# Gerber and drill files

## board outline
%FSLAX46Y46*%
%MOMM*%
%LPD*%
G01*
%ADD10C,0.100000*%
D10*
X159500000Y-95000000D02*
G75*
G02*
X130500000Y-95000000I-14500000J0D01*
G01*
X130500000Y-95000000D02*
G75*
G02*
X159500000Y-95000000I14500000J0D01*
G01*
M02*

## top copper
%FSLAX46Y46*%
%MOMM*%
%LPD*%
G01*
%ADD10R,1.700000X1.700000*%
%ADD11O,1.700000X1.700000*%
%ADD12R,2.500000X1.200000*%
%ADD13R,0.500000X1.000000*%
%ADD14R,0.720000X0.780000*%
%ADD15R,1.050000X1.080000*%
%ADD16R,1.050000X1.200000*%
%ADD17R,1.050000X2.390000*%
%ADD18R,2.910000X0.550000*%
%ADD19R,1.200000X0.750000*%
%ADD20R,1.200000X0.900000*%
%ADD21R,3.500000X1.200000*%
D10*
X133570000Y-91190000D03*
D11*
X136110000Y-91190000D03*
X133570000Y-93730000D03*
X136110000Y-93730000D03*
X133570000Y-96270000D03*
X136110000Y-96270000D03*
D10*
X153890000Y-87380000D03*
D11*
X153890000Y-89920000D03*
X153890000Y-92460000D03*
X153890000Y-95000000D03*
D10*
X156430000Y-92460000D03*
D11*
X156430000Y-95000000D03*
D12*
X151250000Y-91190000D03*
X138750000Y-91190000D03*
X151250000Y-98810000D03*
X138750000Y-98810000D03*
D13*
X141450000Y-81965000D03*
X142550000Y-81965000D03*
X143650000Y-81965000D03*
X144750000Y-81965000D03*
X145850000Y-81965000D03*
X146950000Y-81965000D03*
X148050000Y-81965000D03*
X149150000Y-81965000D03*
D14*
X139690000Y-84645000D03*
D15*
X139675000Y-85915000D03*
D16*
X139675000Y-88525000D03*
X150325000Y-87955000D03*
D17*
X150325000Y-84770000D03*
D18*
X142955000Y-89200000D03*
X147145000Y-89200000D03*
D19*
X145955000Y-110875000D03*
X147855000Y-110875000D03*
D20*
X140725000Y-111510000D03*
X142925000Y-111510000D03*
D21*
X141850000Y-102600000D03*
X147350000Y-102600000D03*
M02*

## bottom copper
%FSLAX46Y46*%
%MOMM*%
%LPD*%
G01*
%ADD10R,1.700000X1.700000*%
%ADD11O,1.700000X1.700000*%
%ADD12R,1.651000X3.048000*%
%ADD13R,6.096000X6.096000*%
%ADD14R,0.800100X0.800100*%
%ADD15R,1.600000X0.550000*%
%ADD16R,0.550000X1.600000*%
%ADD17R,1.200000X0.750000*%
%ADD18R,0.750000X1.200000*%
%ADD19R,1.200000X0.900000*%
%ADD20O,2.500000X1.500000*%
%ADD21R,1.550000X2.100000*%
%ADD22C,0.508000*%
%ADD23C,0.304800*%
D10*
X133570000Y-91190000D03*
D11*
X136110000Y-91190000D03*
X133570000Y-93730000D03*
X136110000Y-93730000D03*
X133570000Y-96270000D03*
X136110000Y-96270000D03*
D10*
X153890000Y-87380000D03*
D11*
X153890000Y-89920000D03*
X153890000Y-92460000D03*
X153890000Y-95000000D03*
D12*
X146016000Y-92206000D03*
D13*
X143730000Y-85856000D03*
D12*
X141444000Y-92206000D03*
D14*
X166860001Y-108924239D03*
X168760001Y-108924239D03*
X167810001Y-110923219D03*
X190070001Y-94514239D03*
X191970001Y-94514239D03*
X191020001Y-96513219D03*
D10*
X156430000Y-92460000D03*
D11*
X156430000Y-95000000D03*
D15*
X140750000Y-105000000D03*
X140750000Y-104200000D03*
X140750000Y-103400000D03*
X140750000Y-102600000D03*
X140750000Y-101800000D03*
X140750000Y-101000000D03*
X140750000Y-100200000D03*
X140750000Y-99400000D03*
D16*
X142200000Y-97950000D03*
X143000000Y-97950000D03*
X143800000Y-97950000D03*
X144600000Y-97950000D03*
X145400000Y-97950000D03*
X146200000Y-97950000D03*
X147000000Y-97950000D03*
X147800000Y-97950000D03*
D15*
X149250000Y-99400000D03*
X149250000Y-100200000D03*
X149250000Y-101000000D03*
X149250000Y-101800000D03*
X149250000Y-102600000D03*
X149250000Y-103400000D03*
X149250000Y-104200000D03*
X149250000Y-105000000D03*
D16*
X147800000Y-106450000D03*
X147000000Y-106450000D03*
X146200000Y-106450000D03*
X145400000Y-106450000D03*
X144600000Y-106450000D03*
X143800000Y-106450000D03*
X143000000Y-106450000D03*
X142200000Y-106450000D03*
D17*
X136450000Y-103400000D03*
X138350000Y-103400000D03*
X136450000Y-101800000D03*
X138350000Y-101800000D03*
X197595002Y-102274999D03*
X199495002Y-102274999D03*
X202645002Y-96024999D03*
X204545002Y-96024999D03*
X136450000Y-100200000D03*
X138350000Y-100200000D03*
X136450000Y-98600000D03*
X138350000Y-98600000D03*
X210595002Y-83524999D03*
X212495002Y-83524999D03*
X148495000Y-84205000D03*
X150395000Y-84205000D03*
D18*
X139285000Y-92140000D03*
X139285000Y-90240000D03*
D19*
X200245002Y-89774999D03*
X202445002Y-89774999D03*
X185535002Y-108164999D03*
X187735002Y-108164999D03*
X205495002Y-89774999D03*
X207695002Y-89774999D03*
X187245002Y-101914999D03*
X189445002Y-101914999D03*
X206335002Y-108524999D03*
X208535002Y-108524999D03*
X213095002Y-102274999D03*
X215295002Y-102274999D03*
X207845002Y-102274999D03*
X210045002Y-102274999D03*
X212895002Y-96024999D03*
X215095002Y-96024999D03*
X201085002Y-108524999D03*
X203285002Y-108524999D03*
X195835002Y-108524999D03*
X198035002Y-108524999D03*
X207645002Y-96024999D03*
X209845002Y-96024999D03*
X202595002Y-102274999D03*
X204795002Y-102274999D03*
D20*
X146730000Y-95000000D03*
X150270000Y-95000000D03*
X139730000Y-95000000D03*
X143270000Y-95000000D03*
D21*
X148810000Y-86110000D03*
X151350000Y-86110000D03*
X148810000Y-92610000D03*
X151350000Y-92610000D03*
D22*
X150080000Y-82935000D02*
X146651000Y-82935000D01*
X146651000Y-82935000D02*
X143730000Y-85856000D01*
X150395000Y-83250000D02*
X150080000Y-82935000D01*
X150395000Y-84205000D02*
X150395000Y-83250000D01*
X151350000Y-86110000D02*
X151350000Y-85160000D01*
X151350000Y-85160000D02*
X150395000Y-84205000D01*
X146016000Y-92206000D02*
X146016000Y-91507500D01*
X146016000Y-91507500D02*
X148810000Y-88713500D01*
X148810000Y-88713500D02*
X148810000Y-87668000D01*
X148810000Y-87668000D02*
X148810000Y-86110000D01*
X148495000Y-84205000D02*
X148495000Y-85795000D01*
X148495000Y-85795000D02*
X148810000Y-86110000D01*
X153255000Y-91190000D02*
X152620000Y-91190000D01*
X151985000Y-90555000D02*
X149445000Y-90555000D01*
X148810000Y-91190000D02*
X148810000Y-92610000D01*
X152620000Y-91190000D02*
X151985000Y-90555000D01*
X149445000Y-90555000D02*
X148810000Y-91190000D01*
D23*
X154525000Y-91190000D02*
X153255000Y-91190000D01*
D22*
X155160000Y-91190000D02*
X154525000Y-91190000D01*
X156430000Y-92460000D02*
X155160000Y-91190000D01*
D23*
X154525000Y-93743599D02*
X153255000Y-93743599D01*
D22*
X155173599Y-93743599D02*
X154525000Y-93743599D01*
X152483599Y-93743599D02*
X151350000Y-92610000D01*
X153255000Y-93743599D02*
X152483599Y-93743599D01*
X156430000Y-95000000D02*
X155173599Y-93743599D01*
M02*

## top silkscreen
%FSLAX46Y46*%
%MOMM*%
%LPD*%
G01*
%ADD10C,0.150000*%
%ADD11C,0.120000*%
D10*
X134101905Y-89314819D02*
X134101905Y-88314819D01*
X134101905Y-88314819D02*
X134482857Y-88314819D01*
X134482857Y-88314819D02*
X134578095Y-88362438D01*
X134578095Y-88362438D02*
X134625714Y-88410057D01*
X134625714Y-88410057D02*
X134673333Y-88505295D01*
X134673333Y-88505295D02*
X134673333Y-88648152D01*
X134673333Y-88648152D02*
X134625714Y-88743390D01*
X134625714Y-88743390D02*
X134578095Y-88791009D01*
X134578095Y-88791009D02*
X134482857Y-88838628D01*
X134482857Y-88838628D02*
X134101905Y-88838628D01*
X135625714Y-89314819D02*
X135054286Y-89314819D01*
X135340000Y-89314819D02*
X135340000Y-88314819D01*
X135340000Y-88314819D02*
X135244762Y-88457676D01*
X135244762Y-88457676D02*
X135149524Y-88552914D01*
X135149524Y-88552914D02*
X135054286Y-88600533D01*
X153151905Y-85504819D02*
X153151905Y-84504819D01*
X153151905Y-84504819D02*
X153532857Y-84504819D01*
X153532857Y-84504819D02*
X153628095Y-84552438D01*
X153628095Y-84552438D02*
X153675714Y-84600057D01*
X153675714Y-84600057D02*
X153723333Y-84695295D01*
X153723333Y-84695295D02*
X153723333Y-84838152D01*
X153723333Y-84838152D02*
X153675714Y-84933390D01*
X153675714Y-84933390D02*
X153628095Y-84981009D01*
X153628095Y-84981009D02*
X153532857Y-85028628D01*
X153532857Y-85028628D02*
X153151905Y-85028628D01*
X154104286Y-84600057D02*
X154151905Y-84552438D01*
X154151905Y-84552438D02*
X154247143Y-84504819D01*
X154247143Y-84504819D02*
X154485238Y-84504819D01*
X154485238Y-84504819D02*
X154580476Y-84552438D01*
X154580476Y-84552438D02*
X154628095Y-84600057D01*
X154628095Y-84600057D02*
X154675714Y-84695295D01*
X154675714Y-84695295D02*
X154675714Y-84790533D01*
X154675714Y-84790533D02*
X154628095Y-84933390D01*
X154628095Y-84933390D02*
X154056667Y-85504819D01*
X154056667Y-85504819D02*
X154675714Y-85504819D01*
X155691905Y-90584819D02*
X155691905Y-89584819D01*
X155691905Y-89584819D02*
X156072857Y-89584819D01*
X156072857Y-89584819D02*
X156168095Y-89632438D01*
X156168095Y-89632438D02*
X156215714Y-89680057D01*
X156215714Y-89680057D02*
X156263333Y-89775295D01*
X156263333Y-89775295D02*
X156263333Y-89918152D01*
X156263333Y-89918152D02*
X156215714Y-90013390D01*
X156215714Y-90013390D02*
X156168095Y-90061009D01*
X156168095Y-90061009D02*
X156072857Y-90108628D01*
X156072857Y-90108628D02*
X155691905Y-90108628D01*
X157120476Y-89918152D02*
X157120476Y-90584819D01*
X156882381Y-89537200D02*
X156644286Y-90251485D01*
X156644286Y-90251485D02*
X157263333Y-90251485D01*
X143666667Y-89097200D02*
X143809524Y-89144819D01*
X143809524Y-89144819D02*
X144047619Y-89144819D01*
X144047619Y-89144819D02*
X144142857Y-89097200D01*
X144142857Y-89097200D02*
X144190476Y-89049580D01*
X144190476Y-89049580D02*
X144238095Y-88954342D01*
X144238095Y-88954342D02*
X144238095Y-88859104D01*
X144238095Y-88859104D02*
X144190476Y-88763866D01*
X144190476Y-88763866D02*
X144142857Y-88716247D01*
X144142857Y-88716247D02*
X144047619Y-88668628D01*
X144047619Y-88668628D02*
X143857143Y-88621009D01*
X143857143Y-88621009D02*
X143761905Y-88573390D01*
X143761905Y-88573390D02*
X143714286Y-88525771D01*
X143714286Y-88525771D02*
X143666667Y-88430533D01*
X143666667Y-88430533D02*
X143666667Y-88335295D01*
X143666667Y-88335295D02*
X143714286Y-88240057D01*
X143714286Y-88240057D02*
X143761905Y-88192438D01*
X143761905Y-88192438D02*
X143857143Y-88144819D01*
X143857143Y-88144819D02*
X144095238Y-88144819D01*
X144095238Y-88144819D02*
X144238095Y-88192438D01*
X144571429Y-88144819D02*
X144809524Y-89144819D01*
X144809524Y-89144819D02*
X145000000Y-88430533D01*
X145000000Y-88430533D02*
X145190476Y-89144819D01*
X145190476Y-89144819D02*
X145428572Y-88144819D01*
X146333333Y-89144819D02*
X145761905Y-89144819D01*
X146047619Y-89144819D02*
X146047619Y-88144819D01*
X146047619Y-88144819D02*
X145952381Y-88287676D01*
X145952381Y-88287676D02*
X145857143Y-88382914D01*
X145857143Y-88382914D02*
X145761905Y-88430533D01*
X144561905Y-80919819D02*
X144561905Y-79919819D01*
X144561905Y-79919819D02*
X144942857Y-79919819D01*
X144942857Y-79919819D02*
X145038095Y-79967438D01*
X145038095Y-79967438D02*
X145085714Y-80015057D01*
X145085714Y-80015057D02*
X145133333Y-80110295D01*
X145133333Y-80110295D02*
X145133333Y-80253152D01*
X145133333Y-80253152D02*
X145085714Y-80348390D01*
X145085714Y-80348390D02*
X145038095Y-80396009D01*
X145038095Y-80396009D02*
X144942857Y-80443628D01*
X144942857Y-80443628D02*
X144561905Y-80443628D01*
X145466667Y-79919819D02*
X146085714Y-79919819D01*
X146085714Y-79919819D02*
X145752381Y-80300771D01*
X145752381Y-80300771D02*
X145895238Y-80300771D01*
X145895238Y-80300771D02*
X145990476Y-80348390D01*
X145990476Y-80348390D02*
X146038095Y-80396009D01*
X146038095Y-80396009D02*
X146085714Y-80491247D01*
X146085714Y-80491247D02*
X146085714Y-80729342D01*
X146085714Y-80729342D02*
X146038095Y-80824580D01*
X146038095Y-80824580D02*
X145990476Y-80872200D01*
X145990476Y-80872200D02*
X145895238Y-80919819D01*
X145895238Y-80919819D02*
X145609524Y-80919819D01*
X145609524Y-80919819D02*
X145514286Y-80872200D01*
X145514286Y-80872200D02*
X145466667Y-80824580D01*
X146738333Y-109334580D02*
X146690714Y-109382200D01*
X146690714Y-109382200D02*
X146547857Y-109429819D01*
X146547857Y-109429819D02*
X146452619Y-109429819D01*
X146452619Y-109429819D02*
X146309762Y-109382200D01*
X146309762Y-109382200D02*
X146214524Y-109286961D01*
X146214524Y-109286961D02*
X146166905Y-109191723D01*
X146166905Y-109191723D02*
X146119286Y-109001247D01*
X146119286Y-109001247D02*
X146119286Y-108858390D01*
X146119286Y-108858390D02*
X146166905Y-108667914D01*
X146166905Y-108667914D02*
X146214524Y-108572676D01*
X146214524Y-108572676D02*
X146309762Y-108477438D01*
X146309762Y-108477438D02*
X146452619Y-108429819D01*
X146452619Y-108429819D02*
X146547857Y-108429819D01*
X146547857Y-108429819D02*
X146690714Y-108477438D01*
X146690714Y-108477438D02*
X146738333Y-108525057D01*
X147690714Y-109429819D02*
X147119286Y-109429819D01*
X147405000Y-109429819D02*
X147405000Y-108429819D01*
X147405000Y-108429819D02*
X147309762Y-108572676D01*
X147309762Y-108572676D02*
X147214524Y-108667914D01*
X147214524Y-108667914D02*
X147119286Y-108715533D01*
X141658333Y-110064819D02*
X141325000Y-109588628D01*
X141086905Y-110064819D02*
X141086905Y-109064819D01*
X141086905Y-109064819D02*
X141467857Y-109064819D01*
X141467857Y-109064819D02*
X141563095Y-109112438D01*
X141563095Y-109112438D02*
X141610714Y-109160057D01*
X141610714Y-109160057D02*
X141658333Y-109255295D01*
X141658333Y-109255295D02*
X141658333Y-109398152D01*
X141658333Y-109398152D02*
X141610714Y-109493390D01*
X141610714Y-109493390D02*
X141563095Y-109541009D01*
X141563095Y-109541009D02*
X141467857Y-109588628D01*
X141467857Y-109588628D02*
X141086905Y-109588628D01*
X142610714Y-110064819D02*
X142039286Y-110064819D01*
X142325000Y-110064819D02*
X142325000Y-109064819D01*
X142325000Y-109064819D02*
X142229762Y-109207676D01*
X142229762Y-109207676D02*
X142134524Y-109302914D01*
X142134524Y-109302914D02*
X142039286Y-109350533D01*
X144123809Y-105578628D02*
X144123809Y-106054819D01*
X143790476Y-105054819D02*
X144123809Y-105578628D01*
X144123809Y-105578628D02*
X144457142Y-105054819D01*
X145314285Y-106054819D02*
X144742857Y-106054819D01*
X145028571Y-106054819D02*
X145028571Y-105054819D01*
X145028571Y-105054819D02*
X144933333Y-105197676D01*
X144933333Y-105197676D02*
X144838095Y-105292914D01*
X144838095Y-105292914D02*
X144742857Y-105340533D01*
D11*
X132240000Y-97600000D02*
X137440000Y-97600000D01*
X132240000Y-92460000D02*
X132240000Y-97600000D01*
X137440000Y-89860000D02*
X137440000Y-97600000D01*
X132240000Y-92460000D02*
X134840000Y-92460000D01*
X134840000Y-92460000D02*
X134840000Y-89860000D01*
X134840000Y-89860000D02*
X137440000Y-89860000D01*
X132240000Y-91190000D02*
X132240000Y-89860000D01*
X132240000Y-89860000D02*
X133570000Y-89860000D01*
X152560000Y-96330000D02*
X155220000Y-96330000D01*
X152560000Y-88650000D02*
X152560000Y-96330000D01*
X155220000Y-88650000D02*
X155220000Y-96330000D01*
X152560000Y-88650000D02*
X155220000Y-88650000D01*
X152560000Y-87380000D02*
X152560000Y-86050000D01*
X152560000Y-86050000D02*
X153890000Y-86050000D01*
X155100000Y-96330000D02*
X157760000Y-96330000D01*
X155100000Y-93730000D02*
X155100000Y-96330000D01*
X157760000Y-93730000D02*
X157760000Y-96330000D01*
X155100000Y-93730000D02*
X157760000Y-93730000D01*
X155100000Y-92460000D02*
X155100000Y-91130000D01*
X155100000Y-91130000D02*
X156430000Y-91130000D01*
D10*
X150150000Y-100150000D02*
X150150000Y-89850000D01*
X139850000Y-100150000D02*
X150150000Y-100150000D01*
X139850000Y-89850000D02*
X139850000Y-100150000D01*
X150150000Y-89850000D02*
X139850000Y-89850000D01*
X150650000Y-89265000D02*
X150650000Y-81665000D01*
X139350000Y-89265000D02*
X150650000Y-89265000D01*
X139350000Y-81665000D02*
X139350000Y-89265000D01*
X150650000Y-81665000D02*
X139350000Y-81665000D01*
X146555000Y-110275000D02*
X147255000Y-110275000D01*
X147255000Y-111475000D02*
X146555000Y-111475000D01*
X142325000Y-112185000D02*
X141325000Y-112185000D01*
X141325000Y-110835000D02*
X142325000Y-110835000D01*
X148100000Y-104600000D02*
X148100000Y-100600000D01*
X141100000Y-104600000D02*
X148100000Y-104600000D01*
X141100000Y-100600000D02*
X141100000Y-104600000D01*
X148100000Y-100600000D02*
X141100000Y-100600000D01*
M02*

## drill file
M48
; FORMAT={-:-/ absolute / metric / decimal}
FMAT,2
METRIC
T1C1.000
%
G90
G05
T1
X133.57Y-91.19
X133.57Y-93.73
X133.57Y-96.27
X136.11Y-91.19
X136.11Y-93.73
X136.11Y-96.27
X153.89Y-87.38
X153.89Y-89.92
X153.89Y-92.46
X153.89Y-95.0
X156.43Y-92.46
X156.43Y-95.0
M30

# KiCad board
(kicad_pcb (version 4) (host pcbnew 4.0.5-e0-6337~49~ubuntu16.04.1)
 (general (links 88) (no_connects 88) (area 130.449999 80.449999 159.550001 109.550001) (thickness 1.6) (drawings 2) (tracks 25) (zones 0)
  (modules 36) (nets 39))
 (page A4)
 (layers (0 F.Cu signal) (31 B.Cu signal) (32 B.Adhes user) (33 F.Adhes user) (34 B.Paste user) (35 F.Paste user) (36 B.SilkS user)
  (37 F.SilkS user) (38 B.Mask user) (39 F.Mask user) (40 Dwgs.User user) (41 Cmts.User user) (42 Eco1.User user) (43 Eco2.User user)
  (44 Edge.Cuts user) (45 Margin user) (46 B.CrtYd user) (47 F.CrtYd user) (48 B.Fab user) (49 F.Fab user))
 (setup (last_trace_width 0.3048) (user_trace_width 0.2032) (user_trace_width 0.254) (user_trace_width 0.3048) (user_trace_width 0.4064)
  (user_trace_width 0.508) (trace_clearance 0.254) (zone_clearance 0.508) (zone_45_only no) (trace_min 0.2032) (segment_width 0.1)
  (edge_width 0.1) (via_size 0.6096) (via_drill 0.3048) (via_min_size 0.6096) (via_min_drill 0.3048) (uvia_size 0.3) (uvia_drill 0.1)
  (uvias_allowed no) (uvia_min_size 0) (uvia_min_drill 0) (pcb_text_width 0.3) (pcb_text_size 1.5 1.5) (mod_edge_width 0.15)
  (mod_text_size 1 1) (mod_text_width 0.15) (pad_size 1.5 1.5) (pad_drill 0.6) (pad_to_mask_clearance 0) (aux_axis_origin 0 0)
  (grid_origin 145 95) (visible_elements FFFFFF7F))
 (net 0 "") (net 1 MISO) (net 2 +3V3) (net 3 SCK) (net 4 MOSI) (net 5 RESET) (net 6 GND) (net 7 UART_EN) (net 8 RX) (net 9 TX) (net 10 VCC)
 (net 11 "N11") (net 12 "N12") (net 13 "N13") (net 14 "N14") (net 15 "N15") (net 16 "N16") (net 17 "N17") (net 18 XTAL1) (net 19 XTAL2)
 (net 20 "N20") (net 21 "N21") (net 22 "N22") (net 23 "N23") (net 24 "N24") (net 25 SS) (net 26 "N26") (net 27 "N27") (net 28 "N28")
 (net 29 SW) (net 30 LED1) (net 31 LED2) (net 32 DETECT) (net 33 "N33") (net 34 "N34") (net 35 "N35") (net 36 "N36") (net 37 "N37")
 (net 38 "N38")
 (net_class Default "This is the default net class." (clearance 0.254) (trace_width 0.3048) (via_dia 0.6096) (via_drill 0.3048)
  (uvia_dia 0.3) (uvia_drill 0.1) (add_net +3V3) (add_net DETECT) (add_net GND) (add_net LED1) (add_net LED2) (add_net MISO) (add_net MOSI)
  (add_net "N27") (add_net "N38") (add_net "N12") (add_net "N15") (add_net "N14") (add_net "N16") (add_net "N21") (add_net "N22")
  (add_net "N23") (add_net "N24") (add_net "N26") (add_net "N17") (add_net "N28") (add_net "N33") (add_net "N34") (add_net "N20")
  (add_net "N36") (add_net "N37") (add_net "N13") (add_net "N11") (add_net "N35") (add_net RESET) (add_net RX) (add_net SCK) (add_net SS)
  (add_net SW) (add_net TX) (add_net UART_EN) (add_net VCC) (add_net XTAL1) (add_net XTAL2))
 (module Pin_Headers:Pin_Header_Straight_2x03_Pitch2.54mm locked (layer F.Cu) (at 133.57 91.19)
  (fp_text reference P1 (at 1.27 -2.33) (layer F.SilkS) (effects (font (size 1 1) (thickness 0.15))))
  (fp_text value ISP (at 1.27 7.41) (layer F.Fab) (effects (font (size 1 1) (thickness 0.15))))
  (fp_line (start -1.33 6.41) (end 3.87 6.41) (layer F.SilkS) (width 0.12))
  (fp_line (start -1.33 1.27) (end -1.33 6.41) (layer F.SilkS) (width 0.12))
  (fp_line (start 3.87 -1.33) (end 3.87 6.41) (layer F.SilkS) (width 0.12))
  (fp_line (start -1.33 1.27) (end 1.27 1.27) (layer F.SilkS) (width 0.12))
  (fp_line (start 1.27 1.27) (end 1.27 -1.33) (layer F.SilkS) (width 0.12))
  (fp_line (start 1.27 -1.33) (end 3.87 -1.33) (layer F.SilkS) (width 0.12))
  (fp_line (start -1.33 0) (end -1.33 -1.33) (layer F.SilkS) (width 0.12))
  (fp_line (start -1.33 -1.33) (end 0 -1.33) (layer F.SilkS) (width 0.12))
  (pad 1 thru_hole rect (at 0 0) (size 1.7 1.7) (drill 1) (layers *.Cu *.Mask) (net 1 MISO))
  (pad 2 thru_hole oval (at 2.54 0) (size 1.7 1.7) (drill 1) (layers *.Cu *.Mask) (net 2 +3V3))
  (pad 3 thru_hole oval (at 0 2.54) (size 1.7 1.7) (drill 1) (layers *.Cu *.Mask) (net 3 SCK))
  (pad 4 thru_hole oval (at 2.54 2.54) (size 1.7 1.7) (drill 1) (layers *.Cu *.Mask) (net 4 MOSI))
  (pad 5 thru_hole oval (at 0 5.08) (size 1.7 1.7) (drill 1) (layers *.Cu *.Mask) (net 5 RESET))
  (pad 6 thru_hole oval (at 2.54 5.08) (size 1.7 1.7) (drill 1) (layers *.Cu *.Mask) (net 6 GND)))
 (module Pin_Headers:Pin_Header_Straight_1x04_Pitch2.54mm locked (layer F.Cu) (at 153.89 87.38)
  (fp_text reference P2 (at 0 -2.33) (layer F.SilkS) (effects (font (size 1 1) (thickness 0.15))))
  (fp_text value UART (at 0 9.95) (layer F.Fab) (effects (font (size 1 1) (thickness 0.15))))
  (fp_line (start -1.33 8.95) (end 1.33 8.95) (layer F.SilkS) (width 0.12))
  (fp_line (start -1.33 1.27) (end -1.33 8.95) (layer F.SilkS) (width 0.12))
  (fp_line (start 1.33 1.27) (end 1.33 8.95) (layer F.SilkS) (width 0.12))
  (fp_line (start -1.33 1.27) (end 1.33 1.27) (layer F.SilkS) (width 0.12))
  (fp_line (start -1.33 0) (end -1.33 -1.33) (layer F.SilkS) (width 0.12))
  (fp_line (start -1.33 -1.33) (end 0 -1.33) (layer F.SilkS) (width 0.12))
  (pad 1 thru_hole rect (at 0 0) (size 1.7 1.7) (drill 1) (layers *.Cu *.Mask) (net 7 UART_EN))
  (pad 2 thru_hole oval (at 0 2.54) (size 1.7 1.7) (drill 1) (layers *.Cu *.Mask) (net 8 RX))
  (pad 3 thru_hole oval (at 0 5.08) (size 1.7 1.7) (drill 1) (layers *.Cu *.Mask) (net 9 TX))
  (pad 4 thru_hole oval (at 0 7.62) (size 1.7 1.7) (drill 1) (layers *.Cu *.Mask) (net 6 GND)))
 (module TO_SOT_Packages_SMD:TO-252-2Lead (layer B.Cu) (at 143.73 92.206 180)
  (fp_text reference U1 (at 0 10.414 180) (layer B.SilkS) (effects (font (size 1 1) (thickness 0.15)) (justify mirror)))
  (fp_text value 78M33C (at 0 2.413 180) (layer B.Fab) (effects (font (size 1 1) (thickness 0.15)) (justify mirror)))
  (pad 1 smd rect (at -2.286 0 180) (size 1.651 3.048) (layers B.Cu B.Paste B.Mask) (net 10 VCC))
  (pad 2 smd rect (at 0 6.35 180) (size 6.096 6.096) (layers B.Cu B.Paste B.Mask) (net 6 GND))
  (pad 3 smd rect (at 2.286 0 180) (size 1.651 3.048) (layers B.Cu B.Paste B.Mask) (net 2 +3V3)))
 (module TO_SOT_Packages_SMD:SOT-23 (layer B.Cu) (at 167.810001 109.924999)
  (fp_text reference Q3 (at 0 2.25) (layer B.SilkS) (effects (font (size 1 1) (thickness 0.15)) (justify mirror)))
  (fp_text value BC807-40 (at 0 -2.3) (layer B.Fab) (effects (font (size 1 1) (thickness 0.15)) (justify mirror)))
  (pad 1 smd rect (at -0.95 -1.00076) (size 0.8001 0.8001) (layers B.Cu B.Paste B.Mask) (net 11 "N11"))
  (pad 2 smd rect (at 0.95 -1.00076) (size 0.8001 0.8001) (layers B.Cu B.Paste B.Mask) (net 2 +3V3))
  (pad 3 smd rect (at 0 0.99822) (size 0.8001 0.8001) (layers B.Cu B.Paste B.Mask) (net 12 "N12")))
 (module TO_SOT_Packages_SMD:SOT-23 (layer B.Cu) (at 191.020001 95.514999)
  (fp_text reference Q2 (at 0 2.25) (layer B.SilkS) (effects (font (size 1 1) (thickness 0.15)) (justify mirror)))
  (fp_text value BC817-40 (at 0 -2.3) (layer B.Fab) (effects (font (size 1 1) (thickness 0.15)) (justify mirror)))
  (pad 1 smd rect (at -0.95 -1.00076) (size 0.8001 0.8001) (layers B.Cu B.Paste B.Mask) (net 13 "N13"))
  (pad 2 smd rect (at 0.95 -1.00076) (size 0.8001 0.8001) (layers B.Cu B.Paste B.Mask) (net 6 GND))
  (pad 3 smd rect (at 0 0.99822) (size 0.8001 0.8001) (layers B.Cu B.Paste B.Mask) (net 8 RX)))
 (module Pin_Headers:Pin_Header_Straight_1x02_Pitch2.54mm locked (layer F.Cu) (at 156.43 92.46)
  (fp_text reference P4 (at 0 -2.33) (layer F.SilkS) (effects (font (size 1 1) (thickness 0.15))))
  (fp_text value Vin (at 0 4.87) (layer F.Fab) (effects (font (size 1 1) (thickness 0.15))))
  (fp_line (start -1.33 3.87) (end 1.33 3.87) (layer F.SilkS) (width 0.12))
  (fp_line (start -1.33 1.27) (end -1.33 3.87) (layer F.SilkS) (width 0.12))
  (fp_line (start 1.33 1.27) (end 1.33 3.87) (layer F.SilkS) (width 0.12))
  (fp_line (start -1.33 1.27) (end 1.33 1.27) (layer F.SilkS) (width 0.12))
  (fp_line (start -1.33 0) (end -1.33 -1.33) (layer F.SilkS) (width 0.12))
  (fp_line (start -1.33 -1.33) (end 0 -1.33) (layer F.SilkS) (width 0.12))
  (pad 1 thru_hole rect (at 0 0) (size 1.7 1.7) (drill 1) (layers *.Cu *.Mask) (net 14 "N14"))
  (pad 2 thru_hole oval (at 0 2.54) (size 1.7 1.7) (drill 1) (layers *.Cu *.Mask) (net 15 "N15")))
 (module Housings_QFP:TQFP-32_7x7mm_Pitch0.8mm (layer B.Cu) (at 145 102.2)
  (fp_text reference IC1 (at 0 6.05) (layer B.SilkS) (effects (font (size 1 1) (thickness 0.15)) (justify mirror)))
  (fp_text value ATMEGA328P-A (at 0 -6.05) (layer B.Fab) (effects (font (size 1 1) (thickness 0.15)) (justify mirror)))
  (pad 1 smd rect (at -4.25 2.8) (size 1.6 0.55) (layers B.Cu B.Paste B.Mask) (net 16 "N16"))
  (pad 2 smd rect (at -4.25 2) (size 1.6 0.55) (layers B.Cu B.Paste B.Mask) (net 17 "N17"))
  (pad 3 smd rect (at -4.25 1.2) (size 1.6 0.55) (layers B.Cu B.Paste B.Mask) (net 6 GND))
  (pad 4 smd rect (at -4.25 0.4) (size 1.6 0.55) (layers B.Cu B.Paste B.Mask) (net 2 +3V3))
  (pad 5 smd rect (at -4.25 -0.4) (size 1.6 0.55) (layers B.Cu B.Paste B.Mask) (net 6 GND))
  (pad 6 smd rect (at -4.25 -1.2) (size 1.6 0.55) (layers B.Cu B.Paste B.Mask) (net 2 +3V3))
  (pad 7 smd rect (at -4.25 -2) (size 1.6 0.55) (layers B.Cu B.Paste B.Mask) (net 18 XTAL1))
  (pad 8 smd rect (at -4.25 -2.8) (size 1.6 0.55) (layers B.Cu B.Paste B.Mask) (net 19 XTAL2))
  (pad 9 smd rect (at -2.8 -4.25 270) (size 1.6 0.55) (layers B.Cu B.Paste B.Mask) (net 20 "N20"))
  (pad 10 smd rect (at -2 -4.25 270) (size 1.6 0.55) (layers B.Cu B.Paste B.Mask) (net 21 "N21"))
  (pad 11 smd rect (at -1.2 -4.25 270) (size 1.6 0.55) (layers B.Cu B.Paste B.Mask) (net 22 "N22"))
  (pad 12 smd rect (at -0.4 -4.25 270) (size 1.6 0.55) (layers B.Cu B.Paste B.Mask) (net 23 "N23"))
  (pad 13 smd rect (at 0.4 -4.25 270) (size 1.6 0.55) (layers B.Cu B.Paste B.Mask) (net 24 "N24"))
  (pad 14 smd rect (at 1.2 -4.25 270) (size 1.6 0.55) (layers B.Cu B.Paste B.Mask) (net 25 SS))
  (pad 15 smd rect (at 2 -4.25 270) (size 1.6 0.55) (layers B.Cu B.Paste B.Mask) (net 4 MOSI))
  (pad 16 smd rect (at 2.8 -4.25 270) (size 1.6 0.55) (layers B.Cu B.Paste B.Mask) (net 1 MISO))
  (pad 17 smd rect (at 4.25 -2.8) (size 1.6 0.55) (layers B.Cu B.Paste B.Mask) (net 3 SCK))
  (pad 18 smd rect (at 4.25 -2) (size 1.6 0.55) (layers B.Cu B.Paste B.Mask) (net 2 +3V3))
  (pad 19 smd rect (at 4.25 -1.2) (size 1.6 0.55) (layers B.Cu B.Paste B.Mask) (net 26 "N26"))
  (pad 20 smd rect (at 4.25 -0.4) (size 1.6 0.55) (layers B.Cu B.Paste B.Mask) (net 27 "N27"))
  (pad 21 smd rect (at 4.25 0.4) (size 1.6 0.55) (layers B.Cu B.Paste B.Mask) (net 6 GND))
  (pad 22 smd rect (at 4.25 1.2) (size 1.6 0.55) (layers B.Cu B.Paste B.Mask) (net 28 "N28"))
  (pad 23 smd rect (at 4.25 2) (size 1.6 0.55) (layers B.Cu B.Paste B.Mask) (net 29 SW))
  (pad 24 smd rect (at 4.25 2.8) (size 1.6 0.55) (layers B.Cu B.Paste B.Mask) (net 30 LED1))
  (pad 25 smd rect (at 2.8 4.25 270) (size 1.6 0.55) (layers B.Cu B.Paste B.Mask) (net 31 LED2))
  (pad 26 smd rect (at 2 4.25 270) (size 1.6 0.55) (layers B.Cu B.Paste B.Mask) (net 7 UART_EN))
  (pad 27 smd rect (at 1.2 4.25 270) (size 1.6 0.55) (layers B.Cu B.Paste B.Mask) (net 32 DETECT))
  (pad 28 smd rect (at 0.4 4.25 270) (size 1.6 0.55) (layers B.Cu B.Paste B.Mask) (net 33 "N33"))
  (pad 29 smd rect (at -0.4 4.25 270) (size 1.6 0.55) (layers B.Cu B.Paste B.Mask) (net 5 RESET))
  (pad 30 smd rect (at -1.2 4.25 270) (size 1.6 0.55) (layers B.Cu B.Paste B.Mask) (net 8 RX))
  (pad 31 smd rect (at -2 4.25 270) (size 1.6 0.55) (layers B.Cu B.Paste B.Mask) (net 9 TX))
  (pad 32 smd rect (at -2.8 4.25 270) (size 1.6 0.55) (layers B.Cu B.Paste B.Mask) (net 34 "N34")))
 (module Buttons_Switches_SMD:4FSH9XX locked (layer F.Cu) (at 145 95)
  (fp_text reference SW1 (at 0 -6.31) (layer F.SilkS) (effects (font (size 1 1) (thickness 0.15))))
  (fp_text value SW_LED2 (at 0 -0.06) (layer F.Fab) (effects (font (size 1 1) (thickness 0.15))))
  (fp_line (start 5.15 5.15) (end 5.15 -5.15) (layer F.SilkS) (width 0.15))
  (fp_line (start -5.15 5.15) (end 5.15 5.15) (layer F.SilkS) (width 0.15))
  (fp_line (start -5.15 -5.15) (end -5.15 5.15) (layer F.SilkS) (width 0.15))
  (fp_line (start 5.15 -5.15) (end -5.15 -5.15) (layer F.SilkS) (width 0.15))
  (pad 1 smd rect (at 6.25 -3.81) (size 2.5 1.2) (layers F.Cu F.Paste F.Mask) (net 29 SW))
  (pad 2 smd rect (at -6.25 -3.81) (size 2.5 1.2) (layers F.Cu F.Paste F.Mask) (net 31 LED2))
  (pad 3 smd rect (at 6.25 3.81) (size 2.5 1.2) (layers F.Cu F.Paste F.Mask) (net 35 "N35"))
  (pad 4 smd rect (at -6.25 3.81) (size 2.5 1.2) (layers F.Cu F.Paste F.Mask) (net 6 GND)))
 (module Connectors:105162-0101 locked (layer F.Cu) (at 145 81.665 180)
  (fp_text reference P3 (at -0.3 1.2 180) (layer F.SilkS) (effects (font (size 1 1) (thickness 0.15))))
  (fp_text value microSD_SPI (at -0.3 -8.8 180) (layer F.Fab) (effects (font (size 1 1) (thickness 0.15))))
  (fp_line (start -5.65 -7.6) (end -5.65 0) (layer F.SilkS) (width 0.15))
  (fp_line (start 5.65 -7.6) (end -5.65 -7.6) (layer F.SilkS) (width 0.15))
  (fp_line (start 5.65 0) (end 5.65 -7.6) (layer F.SilkS) (width 0.15))
  (fp_line (start -5.65 0) (end 5.65 0) (layer F.SilkS) (width 0.15))
  (pad 1 smd rect (at 3.55 -0.3 180) (size 0.5 1) (layers F.Cu F.Paste F.Mask) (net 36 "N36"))
  (pad 2 smd rect (at 2.45 -0.3 180) (size 0.5 1) (layers F.Cu F.Paste F.Mask) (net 25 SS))
  (pad 3 smd rect (at 1.35 -0.3 180) (size 0.5 1) (layers F.Cu F.Paste F.Mask) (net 4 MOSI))
  (pad 4 smd rect (at 0.25 -0.3 180) (size 0.5 1) (layers F.Cu F.Paste F.Mask) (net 2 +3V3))
  (pad 5 smd rect (at -0.85 -0.3 180) (size 0.5 1) (layers F.Cu F.Paste F.Mask) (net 3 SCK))
  (pad 6 smd rect (at -1.95 -0.3 180) (size 0.5 1) (layers F.Cu F.Paste F.Mask) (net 6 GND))
  (pad 7 smd rect (at -3.05 -0.3 180) (size 0.5 1) (layers F.Cu F.Paste F.Mask) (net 1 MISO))
  (pad 8 smd rect (at -4.15 -0.3 180) (size 0.5 1) (layers F.Cu F.Paste F.Mask) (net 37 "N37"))
  (pad 9 smd rect (at 5.31 -2.98 180) (size 0.72 0.78) (layers F.Cu F.Paste F.Mask) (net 32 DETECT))
  (pad G1 smd rect (at 5.325 -4.25 180) (size 1.05 1.08) (layers F.Cu F.Paste F.Mask) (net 6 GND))
  (pad G2 smd rect (at 5.325 -6.86 180) (size 1.05 1.2) (layers F.Cu F.Paste F.Mask) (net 6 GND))
  (pad G3 smd rect (at -5.325 -6.29 180) (size 1.05 1.2) (layers F.Cu F.Paste F.Mask) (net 6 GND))
  (pad G4 smd rect (at -5.325 -3.105 180) (size 1.05 2.39) (layers F.Cu F.Paste F.Mask) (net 6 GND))
  (pad "" smd rect (at 2.045 -7.535 180) (size 2.91 0.55) (layers F.Cu F.Paste F.Mask))
  (pad "" smd rect (at -2.145 -7.535 180) (size 2.91 0.55) (layers F.Cu F.Paste F.Mask)))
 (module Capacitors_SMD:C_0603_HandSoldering (layer F.Cu) (at 146.905 110.875)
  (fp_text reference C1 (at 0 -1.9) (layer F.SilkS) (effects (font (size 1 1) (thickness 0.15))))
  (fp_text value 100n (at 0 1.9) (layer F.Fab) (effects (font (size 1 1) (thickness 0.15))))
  (fp_line (start -0.35 -0.6) (end 0.35 -0.6) (layer F.SilkS) (width 0.15))
  (fp_line (start 0.35 0.6) (end -0.35 0.6) (layer F.SilkS) (width 0.15))
  (pad 1 smd rect (at -0.95 0) (size 1.2 0.75) (layers F.Cu F.Paste F.Mask) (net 5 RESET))
  (pad 2 smd rect (at 0.95 0) (size 1.2 0.75) (layers F.Cu F.Paste F.Mask) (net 6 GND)))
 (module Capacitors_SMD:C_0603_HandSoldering (layer B.Cu) (at 137.4 103.4)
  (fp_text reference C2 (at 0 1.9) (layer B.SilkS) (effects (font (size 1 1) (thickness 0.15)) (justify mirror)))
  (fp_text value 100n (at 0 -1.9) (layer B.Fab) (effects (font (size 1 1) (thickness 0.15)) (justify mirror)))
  (pad 1 smd rect (at -0.95 0) (size 1.2 0.75) (layers B.Cu B.Paste B.Mask) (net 2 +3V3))
  (pad 2 smd rect (at 0.95 0) (size 1.2 0.75) (layers B.Cu B.Paste B.Mask) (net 6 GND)))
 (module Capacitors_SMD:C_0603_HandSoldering (layer B.Cu) (at 137.4 101.8)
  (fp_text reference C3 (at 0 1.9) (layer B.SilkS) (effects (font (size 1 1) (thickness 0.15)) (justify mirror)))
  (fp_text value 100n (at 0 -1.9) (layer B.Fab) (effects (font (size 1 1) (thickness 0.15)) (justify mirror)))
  (pad 1 smd rect (at -0.95 0) (size 1.2 0.75) (layers B.Cu B.Paste B.Mask) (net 2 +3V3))
  (pad 2 smd rect (at 0.95 0) (size 1.2 0.75) (layers B.Cu B.Paste B.Mask) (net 6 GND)))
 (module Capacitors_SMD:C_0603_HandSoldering (layer B.Cu) (at 198.545002 102.274999)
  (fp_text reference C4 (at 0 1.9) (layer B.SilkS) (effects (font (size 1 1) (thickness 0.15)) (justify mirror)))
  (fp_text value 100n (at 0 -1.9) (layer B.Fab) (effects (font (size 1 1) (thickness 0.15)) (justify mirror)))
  (pad 1 smd rect (at -0.95 0) (size 1.2 0.75) (layers B.Cu B.Paste B.Mask) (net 2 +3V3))
  (pad 2 smd rect (at 0.95 0) (size 1.2 0.75) (layers B.Cu B.Paste B.Mask) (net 6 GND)))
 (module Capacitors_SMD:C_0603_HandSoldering (layer B.Cu) (at 203.595002 96.024999)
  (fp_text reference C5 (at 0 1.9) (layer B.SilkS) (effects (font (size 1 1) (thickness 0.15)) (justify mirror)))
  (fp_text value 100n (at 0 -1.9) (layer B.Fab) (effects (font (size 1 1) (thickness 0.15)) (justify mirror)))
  (pad 1 smd rect (at -0.95 0) (size 1.2 0.75) (layers B.Cu B.Paste B.Mask) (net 27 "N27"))
  (pad 2 smd rect (at 0.95 0) (size 1.2 0.75) (layers B.Cu B.Paste B.Mask) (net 6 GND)))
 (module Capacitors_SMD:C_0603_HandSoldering (layer B.Cu) (at 137.4 100.2)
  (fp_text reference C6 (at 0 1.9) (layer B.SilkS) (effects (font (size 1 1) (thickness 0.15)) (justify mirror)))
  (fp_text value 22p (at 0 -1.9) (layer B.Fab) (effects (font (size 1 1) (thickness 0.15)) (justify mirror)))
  (pad 1 smd rect (at -0.95 0) (size 1.2 0.75) (layers B.Cu B.Paste B.Mask) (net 6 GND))
  (pad 2 smd rect (at 0.95 0) (size 1.2 0.75) (layers B.Cu B.Paste B.Mask) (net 18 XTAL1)))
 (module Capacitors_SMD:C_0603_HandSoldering (layer B.Cu) (at 137.4 98.6)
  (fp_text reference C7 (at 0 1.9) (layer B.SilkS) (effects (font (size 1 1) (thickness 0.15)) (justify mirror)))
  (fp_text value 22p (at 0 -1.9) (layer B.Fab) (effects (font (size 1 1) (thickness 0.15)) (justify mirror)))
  (pad 1 smd rect (at -0.95 0) (size 1.2 0.75) (layers B.Cu B.Paste B.Mask) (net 6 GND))
  (pad 2 smd rect (at 0.95 0) (size 1.2 0.75) (layers B.Cu B.Paste B.Mask) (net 19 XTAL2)))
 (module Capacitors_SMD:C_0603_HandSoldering (layer B.Cu) (at 211.545002 83.524999)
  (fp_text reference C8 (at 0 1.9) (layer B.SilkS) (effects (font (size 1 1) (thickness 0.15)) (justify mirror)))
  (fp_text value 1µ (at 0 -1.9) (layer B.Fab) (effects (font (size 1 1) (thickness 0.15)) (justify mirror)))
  (pad 1 smd rect (at -0.95 0) (size 1.2 0.75) (layers B.Cu B.Paste B.Mask) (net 2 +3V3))
  (pad 2 smd rect (at 0.95 0) (size 1.2 0.75) (layers B.Cu B.Paste B.Mask) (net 6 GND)))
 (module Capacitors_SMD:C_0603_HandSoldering (layer B.Cu) (at 149.445 84.205)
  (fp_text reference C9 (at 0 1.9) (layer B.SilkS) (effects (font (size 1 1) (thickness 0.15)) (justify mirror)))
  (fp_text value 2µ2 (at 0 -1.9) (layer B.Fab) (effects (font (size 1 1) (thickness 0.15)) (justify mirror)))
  (pad 1 smd rect (at -0.95 0) (size 1.2 0.75) (layers B.Cu B.Paste B.Mask) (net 10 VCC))
  (pad 2 smd rect (at 0.95 0) (size 1.2 0.75) (layers B.Cu B.Paste B.Mask) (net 6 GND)))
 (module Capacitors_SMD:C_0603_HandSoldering (layer B.Cu) (at 139.285 91.19 90)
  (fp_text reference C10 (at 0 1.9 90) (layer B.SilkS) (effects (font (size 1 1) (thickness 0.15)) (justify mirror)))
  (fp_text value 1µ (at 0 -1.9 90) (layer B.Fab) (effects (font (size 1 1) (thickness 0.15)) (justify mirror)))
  (pad 1 smd rect (at -0.95 0 90) (size 1.2 0.75) (layers B.Cu B.Paste B.Mask) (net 2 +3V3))
  (pad 2 smd rect (at 0.95 0 90) (size 1.2 0.75) (layers B.Cu B.Paste B.Mask) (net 6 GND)))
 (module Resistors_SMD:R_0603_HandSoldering (layer F.Cu) (at 141.825 111.51)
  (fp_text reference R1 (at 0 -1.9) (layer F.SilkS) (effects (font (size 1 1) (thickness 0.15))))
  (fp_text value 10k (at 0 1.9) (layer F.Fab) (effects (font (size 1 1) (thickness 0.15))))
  (fp_line (start 0.5 0.675) (end -0.5 0.675) (layer F.SilkS) (width 0.15))
  (fp_line (start -0.5 -0.675) (end 0.5 -0.675) (layer F.SilkS) (width 0.15))
  (pad 1 smd rect (at -1.1 0) (size 1.2 0.9) (layers F.Cu F.Paste F.Mask) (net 2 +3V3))
  (pad 2 smd rect (at 1.1 0) (size 1.2 0.9) (layers F.Cu F.Paste F.Mask) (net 5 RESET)))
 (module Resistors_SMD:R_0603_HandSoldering (layer B.Cu) (at 201.345002 89.774999)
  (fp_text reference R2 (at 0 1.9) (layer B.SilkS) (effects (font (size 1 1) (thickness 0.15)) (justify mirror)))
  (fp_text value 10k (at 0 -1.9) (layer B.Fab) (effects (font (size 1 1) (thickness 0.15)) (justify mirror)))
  (pad 1 smd rect (at -1.1 0) (size 1.2 0.9) (layers B.Cu B.Paste B.Mask) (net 2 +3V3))
  (pad 2 smd rect (at 1.1 0) (size 1.2 0.9) (layers B.Cu B.Paste B.Mask) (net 7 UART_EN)))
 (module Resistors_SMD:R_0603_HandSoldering (layer B.Cu) (at 186.635002 108.164999)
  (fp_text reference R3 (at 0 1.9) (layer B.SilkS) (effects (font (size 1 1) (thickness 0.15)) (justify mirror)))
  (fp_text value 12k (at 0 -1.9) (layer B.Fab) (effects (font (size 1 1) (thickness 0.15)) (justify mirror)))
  (pad 1 smd rect (at -1.1 0) (size 1.2 0.9) (layers B.Cu B.Paste B.Mask) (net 13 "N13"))
  (pad 2 smd rect (at 1.1 0) (size 1.2 0.9) (layers B.Cu B.Paste B.Mask) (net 6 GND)))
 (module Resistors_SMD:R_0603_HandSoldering (layer B.Cu) (at 206.595002 89.774999)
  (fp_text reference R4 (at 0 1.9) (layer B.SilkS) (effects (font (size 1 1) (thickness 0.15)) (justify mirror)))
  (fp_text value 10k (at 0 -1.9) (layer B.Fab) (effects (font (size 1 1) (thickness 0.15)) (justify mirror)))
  (pad 1 smd rect (at -1.1 0) (size 1.2 0.9) (layers B.Cu B.Paste B.Mask) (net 2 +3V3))
  (pad 2 smd rect (at 1.1 0) (size 1.2 0.9) (layers B.Cu B.Paste B.Mask) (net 1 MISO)))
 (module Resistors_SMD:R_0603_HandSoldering (layer B.Cu) (at 188.345002 101.914999)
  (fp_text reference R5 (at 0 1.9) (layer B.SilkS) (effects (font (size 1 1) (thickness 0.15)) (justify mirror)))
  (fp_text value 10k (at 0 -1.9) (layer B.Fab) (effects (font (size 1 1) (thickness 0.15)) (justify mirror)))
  (pad 1 smd rect (at -1.1 0) (size 1.2 0.9) (layers B.Cu B.Paste B.Mask) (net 2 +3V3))
  (pad 2 smd rect (at 1.1 0) (size 1.2 0.9) (layers B.Cu B.Paste B.Mask) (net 25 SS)))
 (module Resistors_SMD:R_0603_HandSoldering (layer B.Cu) (at 207.435002 108.524999)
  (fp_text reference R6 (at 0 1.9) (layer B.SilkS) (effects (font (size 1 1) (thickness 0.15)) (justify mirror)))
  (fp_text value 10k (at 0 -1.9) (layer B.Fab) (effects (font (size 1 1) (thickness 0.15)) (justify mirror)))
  (pad 1 smd rect (at -1.1 0) (size 1.2 0.9) (layers B.Cu B.Paste B.Mask) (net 2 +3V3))
  (pad 2 smd rect (at 1.1 0) (size 1.2 0.9) (layers B.Cu B.Paste B.Mask) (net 32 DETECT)))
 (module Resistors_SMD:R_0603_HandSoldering (layer B.Cu) (at 214.195002 102.274999)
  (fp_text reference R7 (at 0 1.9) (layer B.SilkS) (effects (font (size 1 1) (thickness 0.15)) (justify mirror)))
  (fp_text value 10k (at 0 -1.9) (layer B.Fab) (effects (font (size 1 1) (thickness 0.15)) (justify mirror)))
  (pad 1 smd rect (at -1.1 0) (size 1.2 0.9) (layers B.Cu B.Paste B.Mask) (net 2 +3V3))
  (pad 2 smd rect (at 1.1 0) (size 1.2 0.9) (layers B.Cu B.Paste B.Mask) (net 37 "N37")))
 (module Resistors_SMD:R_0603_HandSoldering (layer B.Cu) (at 208.945002 102.274999)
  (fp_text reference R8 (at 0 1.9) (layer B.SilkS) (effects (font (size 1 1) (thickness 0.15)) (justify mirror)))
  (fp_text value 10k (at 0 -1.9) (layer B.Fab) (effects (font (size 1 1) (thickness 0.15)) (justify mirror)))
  (pad 1 smd rect (at -1.1 0) (size 1.2 0.9) (layers B.Cu B.Paste B.Mask) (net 2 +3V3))
  (pad 2 smd rect (at 1.1 0) (size 1.2 0.9) (layers B.Cu B.Paste B.Mask) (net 36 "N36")))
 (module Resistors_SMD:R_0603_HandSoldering (layer B.Cu) (at 213.995002 96.024999)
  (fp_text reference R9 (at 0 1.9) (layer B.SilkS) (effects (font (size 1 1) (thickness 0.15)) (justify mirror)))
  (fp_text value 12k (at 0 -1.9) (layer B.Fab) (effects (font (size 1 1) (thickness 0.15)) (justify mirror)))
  (pad 1 smd rect (at -1.1 0) (size 1.2 0.9) (layers B.Cu B.Paste B.Mask) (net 2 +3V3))
  (pad 2 smd rect (at 1.1 0) (size 1.2 0.9) (layers B.Cu B.Paste B.Mask) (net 8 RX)))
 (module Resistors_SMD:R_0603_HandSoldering (layer B.Cu) (at 202.185002 108.524999)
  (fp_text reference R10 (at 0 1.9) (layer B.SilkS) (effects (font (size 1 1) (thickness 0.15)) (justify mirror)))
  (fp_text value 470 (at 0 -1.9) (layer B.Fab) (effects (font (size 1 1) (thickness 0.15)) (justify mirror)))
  (pad 1 smd rect (at -1.1 0) (size 1.2 0.9) (layers B.Cu B.Paste B.Mask) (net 30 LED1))
  (pad 2 smd rect (at 1.1 0) (size 1.2 0.9) (layers B.Cu B.Paste B.Mask) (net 35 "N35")))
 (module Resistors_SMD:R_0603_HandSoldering (layer B.Cu) (at 196.935002 108.524999)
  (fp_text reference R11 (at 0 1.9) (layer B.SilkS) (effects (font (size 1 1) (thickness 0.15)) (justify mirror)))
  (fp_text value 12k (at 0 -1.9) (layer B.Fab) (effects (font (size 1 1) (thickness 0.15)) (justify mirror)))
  (pad 1 smd rect (at -1.1 0) (size 1.2 0.9) (layers B.Cu B.Paste B.Mask) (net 11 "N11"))
  (pad 2 smd rect (at 1.1 0) (size 1.2 0.9) (layers B.Cu B.Paste B.Mask) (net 9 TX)))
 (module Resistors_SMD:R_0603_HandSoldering (layer B.Cu) (at 208.745002 96.024999)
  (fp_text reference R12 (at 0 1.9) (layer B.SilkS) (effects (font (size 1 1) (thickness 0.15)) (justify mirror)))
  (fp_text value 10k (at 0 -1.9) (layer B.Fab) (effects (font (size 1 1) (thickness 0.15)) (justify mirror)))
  (pad 1 smd rect (at -1.1 0) (size 1.2 0.9) (layers B.Cu B.Paste B.Mask) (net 2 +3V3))
  (pad 2 smd rect (at 1.1 0) (size 1.2 0.9) (layers B.Cu B.Paste B.Mask) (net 29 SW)))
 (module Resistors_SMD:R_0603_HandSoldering (layer B.Cu) (at 203.695002 102.274999)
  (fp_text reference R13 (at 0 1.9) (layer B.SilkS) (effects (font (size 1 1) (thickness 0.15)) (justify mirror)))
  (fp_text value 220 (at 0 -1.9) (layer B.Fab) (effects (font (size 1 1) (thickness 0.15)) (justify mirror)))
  (pad 1 smd rect (at -1.1 0) (size 1.2 0.9) (layers B.Cu B.Paste B.Mask) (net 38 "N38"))
  (pad 2 smd rect (at 1.1 0) (size 1.2 0.9) (layers B.Cu B.Paste B.Mask) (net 6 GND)))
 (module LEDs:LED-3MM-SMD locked (layer B.Cu) (at 148.5 95)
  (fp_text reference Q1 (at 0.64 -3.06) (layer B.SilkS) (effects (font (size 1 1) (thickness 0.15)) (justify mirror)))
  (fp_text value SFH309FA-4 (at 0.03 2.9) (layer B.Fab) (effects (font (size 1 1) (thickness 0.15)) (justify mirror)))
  (pad 1 smd oval (at -1.77 0 270) (size 1.5 2.5) (layers B.Cu B.Paste B.Mask) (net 2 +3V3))
  (pad 2 smd oval (at 1.77 0) (size 2.5 1.5) (layers B.Cu B.Paste B.Mask) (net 13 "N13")))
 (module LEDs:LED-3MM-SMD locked (layer B.Cu) (at 141.5 95)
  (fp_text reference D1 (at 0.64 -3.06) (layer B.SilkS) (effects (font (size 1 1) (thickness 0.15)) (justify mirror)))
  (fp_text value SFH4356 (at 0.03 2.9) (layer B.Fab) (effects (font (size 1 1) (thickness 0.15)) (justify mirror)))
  (pad 1 smd oval (at -1.77 0 270) (size 1.5 2.5) (layers B.Cu B.Paste B.Mask) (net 38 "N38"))
  (pad 2 smd oval (at 1.77 0) (size 2.5 1.5) (layers B.Cu B.Paste B.Mask) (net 12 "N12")))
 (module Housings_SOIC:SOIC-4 (layer B.Cu) (at 150.08 89.36)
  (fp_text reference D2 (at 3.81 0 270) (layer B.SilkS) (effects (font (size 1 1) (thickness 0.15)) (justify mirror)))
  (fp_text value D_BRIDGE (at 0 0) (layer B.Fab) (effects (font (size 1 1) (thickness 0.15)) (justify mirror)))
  (pad 1 smd rect (at -1.27 -3.25) (size 1.55 2.1) (layers B.Cu B.Paste B.Mask) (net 10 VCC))
  (pad 2 smd rect (at 1.27 -3.25) (size 1.55 2.1) (layers B.Cu B.Paste B.Mask) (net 6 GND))
  (pad 4 smd rect (at -1.27 3.25) (size 1.55 2.1) (layers B.Cu B.Paste B.Mask) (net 14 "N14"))
  (pad 3 smd rect (at 1.27 3.25) (size 1.55 2.1) (layers B.Cu B.Paste B.Mask) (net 15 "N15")))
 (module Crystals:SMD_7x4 (layer F.Cu) (at 144.6 102.6)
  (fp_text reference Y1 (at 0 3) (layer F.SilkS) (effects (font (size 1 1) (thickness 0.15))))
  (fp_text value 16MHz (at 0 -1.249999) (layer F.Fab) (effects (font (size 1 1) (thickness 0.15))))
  (fp_line (start 3.5 2) (end 3.5 -2) (layer F.SilkS) (width 0.15))
  (fp_line (start -3.5 2) (end 3.5 2) (layer F.SilkS) (width 0.15))
  (fp_line (start -3.5 -2) (end -3.5 2) (layer F.SilkS) (width 0.15))
  (fp_line (start 3.5 -2) (end -3.5 -2) (layer F.SilkS) (width 0.15))
  (pad 1 smd rect (at -2.75 0) (size 3.5 1.2) (layers F.Cu F.Paste F.Mask) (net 18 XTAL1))
  (pad 2 smd rect (at 2.75 0) (size 3.5 1.2) (layers F.Cu F.Paste F.Mask) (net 19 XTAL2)))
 (gr_circle (center 145 95) (end 159.5 95) (layer Edge.Cuts) (width 0.1))
 (segment (start 150.08 82.935) (end 146.651 82.935) (width 0.508) (layer B.Cu) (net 6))
 (segment (start 146.651 82.935) (end 143.73 85.856) (width 0.508) (layer B.Cu) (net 6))
 (segment (start 150.395 83.25) (end 150.08 82.935) (width 0.508) (layer B.Cu) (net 6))
 (segment (start 150.395 84.205) (end 150.395 83.25) (width 0.508) (layer B.Cu) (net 6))
 (segment (start 151.35 86.11) (end 151.35 85.16) (width 0.508) (layer B.Cu) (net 6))
 (segment (start 151.35 85.16) (end 150.395 84.205) (width 0.508) (layer B.Cu) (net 6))
 (segment (start 146.016 92.206) (end 146.016 91.5075) (width 0.508) (layer B.Cu) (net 10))
 (segment (start 146.016 91.5075) (end 148.81 88.7135) (width 0.508) (layer B.Cu) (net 10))
 (segment (start 148.81 88.7135) (end 148.81 87.668) (width 0.508) (layer B.Cu) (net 10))
 (segment (start 148.81 87.668) (end 148.81 86.11) (width 0.508) (layer B.Cu) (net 10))
 (segment (start 148.495 84.205) (end 148.495 85.795) (width 0.508) (layer B.Cu) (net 10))
 (segment (start 148.495 85.795) (end 148.81 86.11) (width 0.508) (layer B.Cu) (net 10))
 (segment (start 153.255 91.19) (end 152.62 91.19) (width 0.508) (layer B.Cu) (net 14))
 (segment (start 151.985 90.555) (end 149.445 90.555) (width 0.508) (layer B.Cu) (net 14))
 (segment (start 148.81 91.19) (end 148.81 92.61) (width 0.508) (layer B.Cu) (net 14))
 (segment (start 152.62 91.19) (end 151.985 90.555) (width 0.508) (layer B.Cu) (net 14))
 (segment (start 149.445 90.555) (end 148.81 91.19) (width 0.508) (layer B.Cu) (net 14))
 (segment (start 154.525 91.19) (end 153.255 91.19) (width 0.3048) (layer B.Cu) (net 14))
 (segment (start 155.16 91.19) (end 154.525 91.19) (width 0.508) (layer B.Cu) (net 14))
 (segment (start 156.43 92.46) (end 155.16 91.19) (width 0.508) (layer B.Cu) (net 14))
 (segment (start 154.525 93.743599) (end 153.255 93.743599) (width 0.3048) (layer B.Cu) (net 15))
 (segment (start 155.173599 93.743599) (end 154.525 93.743599) (width 0.508) (layer B.Cu) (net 15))
 (segment (start 152.483599 93.743599) (end 151.35 92.61) (width 0.508) (layer B.Cu) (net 15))
 (segment (start 153.255 93.743599) (end 152.483599 93.743599) (width 0.508) (layer B.Cu) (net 15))
 (segment (start 156.43 95) (end 155.173599 93.743599) (width 0.508) (layer B.Cu) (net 15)))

